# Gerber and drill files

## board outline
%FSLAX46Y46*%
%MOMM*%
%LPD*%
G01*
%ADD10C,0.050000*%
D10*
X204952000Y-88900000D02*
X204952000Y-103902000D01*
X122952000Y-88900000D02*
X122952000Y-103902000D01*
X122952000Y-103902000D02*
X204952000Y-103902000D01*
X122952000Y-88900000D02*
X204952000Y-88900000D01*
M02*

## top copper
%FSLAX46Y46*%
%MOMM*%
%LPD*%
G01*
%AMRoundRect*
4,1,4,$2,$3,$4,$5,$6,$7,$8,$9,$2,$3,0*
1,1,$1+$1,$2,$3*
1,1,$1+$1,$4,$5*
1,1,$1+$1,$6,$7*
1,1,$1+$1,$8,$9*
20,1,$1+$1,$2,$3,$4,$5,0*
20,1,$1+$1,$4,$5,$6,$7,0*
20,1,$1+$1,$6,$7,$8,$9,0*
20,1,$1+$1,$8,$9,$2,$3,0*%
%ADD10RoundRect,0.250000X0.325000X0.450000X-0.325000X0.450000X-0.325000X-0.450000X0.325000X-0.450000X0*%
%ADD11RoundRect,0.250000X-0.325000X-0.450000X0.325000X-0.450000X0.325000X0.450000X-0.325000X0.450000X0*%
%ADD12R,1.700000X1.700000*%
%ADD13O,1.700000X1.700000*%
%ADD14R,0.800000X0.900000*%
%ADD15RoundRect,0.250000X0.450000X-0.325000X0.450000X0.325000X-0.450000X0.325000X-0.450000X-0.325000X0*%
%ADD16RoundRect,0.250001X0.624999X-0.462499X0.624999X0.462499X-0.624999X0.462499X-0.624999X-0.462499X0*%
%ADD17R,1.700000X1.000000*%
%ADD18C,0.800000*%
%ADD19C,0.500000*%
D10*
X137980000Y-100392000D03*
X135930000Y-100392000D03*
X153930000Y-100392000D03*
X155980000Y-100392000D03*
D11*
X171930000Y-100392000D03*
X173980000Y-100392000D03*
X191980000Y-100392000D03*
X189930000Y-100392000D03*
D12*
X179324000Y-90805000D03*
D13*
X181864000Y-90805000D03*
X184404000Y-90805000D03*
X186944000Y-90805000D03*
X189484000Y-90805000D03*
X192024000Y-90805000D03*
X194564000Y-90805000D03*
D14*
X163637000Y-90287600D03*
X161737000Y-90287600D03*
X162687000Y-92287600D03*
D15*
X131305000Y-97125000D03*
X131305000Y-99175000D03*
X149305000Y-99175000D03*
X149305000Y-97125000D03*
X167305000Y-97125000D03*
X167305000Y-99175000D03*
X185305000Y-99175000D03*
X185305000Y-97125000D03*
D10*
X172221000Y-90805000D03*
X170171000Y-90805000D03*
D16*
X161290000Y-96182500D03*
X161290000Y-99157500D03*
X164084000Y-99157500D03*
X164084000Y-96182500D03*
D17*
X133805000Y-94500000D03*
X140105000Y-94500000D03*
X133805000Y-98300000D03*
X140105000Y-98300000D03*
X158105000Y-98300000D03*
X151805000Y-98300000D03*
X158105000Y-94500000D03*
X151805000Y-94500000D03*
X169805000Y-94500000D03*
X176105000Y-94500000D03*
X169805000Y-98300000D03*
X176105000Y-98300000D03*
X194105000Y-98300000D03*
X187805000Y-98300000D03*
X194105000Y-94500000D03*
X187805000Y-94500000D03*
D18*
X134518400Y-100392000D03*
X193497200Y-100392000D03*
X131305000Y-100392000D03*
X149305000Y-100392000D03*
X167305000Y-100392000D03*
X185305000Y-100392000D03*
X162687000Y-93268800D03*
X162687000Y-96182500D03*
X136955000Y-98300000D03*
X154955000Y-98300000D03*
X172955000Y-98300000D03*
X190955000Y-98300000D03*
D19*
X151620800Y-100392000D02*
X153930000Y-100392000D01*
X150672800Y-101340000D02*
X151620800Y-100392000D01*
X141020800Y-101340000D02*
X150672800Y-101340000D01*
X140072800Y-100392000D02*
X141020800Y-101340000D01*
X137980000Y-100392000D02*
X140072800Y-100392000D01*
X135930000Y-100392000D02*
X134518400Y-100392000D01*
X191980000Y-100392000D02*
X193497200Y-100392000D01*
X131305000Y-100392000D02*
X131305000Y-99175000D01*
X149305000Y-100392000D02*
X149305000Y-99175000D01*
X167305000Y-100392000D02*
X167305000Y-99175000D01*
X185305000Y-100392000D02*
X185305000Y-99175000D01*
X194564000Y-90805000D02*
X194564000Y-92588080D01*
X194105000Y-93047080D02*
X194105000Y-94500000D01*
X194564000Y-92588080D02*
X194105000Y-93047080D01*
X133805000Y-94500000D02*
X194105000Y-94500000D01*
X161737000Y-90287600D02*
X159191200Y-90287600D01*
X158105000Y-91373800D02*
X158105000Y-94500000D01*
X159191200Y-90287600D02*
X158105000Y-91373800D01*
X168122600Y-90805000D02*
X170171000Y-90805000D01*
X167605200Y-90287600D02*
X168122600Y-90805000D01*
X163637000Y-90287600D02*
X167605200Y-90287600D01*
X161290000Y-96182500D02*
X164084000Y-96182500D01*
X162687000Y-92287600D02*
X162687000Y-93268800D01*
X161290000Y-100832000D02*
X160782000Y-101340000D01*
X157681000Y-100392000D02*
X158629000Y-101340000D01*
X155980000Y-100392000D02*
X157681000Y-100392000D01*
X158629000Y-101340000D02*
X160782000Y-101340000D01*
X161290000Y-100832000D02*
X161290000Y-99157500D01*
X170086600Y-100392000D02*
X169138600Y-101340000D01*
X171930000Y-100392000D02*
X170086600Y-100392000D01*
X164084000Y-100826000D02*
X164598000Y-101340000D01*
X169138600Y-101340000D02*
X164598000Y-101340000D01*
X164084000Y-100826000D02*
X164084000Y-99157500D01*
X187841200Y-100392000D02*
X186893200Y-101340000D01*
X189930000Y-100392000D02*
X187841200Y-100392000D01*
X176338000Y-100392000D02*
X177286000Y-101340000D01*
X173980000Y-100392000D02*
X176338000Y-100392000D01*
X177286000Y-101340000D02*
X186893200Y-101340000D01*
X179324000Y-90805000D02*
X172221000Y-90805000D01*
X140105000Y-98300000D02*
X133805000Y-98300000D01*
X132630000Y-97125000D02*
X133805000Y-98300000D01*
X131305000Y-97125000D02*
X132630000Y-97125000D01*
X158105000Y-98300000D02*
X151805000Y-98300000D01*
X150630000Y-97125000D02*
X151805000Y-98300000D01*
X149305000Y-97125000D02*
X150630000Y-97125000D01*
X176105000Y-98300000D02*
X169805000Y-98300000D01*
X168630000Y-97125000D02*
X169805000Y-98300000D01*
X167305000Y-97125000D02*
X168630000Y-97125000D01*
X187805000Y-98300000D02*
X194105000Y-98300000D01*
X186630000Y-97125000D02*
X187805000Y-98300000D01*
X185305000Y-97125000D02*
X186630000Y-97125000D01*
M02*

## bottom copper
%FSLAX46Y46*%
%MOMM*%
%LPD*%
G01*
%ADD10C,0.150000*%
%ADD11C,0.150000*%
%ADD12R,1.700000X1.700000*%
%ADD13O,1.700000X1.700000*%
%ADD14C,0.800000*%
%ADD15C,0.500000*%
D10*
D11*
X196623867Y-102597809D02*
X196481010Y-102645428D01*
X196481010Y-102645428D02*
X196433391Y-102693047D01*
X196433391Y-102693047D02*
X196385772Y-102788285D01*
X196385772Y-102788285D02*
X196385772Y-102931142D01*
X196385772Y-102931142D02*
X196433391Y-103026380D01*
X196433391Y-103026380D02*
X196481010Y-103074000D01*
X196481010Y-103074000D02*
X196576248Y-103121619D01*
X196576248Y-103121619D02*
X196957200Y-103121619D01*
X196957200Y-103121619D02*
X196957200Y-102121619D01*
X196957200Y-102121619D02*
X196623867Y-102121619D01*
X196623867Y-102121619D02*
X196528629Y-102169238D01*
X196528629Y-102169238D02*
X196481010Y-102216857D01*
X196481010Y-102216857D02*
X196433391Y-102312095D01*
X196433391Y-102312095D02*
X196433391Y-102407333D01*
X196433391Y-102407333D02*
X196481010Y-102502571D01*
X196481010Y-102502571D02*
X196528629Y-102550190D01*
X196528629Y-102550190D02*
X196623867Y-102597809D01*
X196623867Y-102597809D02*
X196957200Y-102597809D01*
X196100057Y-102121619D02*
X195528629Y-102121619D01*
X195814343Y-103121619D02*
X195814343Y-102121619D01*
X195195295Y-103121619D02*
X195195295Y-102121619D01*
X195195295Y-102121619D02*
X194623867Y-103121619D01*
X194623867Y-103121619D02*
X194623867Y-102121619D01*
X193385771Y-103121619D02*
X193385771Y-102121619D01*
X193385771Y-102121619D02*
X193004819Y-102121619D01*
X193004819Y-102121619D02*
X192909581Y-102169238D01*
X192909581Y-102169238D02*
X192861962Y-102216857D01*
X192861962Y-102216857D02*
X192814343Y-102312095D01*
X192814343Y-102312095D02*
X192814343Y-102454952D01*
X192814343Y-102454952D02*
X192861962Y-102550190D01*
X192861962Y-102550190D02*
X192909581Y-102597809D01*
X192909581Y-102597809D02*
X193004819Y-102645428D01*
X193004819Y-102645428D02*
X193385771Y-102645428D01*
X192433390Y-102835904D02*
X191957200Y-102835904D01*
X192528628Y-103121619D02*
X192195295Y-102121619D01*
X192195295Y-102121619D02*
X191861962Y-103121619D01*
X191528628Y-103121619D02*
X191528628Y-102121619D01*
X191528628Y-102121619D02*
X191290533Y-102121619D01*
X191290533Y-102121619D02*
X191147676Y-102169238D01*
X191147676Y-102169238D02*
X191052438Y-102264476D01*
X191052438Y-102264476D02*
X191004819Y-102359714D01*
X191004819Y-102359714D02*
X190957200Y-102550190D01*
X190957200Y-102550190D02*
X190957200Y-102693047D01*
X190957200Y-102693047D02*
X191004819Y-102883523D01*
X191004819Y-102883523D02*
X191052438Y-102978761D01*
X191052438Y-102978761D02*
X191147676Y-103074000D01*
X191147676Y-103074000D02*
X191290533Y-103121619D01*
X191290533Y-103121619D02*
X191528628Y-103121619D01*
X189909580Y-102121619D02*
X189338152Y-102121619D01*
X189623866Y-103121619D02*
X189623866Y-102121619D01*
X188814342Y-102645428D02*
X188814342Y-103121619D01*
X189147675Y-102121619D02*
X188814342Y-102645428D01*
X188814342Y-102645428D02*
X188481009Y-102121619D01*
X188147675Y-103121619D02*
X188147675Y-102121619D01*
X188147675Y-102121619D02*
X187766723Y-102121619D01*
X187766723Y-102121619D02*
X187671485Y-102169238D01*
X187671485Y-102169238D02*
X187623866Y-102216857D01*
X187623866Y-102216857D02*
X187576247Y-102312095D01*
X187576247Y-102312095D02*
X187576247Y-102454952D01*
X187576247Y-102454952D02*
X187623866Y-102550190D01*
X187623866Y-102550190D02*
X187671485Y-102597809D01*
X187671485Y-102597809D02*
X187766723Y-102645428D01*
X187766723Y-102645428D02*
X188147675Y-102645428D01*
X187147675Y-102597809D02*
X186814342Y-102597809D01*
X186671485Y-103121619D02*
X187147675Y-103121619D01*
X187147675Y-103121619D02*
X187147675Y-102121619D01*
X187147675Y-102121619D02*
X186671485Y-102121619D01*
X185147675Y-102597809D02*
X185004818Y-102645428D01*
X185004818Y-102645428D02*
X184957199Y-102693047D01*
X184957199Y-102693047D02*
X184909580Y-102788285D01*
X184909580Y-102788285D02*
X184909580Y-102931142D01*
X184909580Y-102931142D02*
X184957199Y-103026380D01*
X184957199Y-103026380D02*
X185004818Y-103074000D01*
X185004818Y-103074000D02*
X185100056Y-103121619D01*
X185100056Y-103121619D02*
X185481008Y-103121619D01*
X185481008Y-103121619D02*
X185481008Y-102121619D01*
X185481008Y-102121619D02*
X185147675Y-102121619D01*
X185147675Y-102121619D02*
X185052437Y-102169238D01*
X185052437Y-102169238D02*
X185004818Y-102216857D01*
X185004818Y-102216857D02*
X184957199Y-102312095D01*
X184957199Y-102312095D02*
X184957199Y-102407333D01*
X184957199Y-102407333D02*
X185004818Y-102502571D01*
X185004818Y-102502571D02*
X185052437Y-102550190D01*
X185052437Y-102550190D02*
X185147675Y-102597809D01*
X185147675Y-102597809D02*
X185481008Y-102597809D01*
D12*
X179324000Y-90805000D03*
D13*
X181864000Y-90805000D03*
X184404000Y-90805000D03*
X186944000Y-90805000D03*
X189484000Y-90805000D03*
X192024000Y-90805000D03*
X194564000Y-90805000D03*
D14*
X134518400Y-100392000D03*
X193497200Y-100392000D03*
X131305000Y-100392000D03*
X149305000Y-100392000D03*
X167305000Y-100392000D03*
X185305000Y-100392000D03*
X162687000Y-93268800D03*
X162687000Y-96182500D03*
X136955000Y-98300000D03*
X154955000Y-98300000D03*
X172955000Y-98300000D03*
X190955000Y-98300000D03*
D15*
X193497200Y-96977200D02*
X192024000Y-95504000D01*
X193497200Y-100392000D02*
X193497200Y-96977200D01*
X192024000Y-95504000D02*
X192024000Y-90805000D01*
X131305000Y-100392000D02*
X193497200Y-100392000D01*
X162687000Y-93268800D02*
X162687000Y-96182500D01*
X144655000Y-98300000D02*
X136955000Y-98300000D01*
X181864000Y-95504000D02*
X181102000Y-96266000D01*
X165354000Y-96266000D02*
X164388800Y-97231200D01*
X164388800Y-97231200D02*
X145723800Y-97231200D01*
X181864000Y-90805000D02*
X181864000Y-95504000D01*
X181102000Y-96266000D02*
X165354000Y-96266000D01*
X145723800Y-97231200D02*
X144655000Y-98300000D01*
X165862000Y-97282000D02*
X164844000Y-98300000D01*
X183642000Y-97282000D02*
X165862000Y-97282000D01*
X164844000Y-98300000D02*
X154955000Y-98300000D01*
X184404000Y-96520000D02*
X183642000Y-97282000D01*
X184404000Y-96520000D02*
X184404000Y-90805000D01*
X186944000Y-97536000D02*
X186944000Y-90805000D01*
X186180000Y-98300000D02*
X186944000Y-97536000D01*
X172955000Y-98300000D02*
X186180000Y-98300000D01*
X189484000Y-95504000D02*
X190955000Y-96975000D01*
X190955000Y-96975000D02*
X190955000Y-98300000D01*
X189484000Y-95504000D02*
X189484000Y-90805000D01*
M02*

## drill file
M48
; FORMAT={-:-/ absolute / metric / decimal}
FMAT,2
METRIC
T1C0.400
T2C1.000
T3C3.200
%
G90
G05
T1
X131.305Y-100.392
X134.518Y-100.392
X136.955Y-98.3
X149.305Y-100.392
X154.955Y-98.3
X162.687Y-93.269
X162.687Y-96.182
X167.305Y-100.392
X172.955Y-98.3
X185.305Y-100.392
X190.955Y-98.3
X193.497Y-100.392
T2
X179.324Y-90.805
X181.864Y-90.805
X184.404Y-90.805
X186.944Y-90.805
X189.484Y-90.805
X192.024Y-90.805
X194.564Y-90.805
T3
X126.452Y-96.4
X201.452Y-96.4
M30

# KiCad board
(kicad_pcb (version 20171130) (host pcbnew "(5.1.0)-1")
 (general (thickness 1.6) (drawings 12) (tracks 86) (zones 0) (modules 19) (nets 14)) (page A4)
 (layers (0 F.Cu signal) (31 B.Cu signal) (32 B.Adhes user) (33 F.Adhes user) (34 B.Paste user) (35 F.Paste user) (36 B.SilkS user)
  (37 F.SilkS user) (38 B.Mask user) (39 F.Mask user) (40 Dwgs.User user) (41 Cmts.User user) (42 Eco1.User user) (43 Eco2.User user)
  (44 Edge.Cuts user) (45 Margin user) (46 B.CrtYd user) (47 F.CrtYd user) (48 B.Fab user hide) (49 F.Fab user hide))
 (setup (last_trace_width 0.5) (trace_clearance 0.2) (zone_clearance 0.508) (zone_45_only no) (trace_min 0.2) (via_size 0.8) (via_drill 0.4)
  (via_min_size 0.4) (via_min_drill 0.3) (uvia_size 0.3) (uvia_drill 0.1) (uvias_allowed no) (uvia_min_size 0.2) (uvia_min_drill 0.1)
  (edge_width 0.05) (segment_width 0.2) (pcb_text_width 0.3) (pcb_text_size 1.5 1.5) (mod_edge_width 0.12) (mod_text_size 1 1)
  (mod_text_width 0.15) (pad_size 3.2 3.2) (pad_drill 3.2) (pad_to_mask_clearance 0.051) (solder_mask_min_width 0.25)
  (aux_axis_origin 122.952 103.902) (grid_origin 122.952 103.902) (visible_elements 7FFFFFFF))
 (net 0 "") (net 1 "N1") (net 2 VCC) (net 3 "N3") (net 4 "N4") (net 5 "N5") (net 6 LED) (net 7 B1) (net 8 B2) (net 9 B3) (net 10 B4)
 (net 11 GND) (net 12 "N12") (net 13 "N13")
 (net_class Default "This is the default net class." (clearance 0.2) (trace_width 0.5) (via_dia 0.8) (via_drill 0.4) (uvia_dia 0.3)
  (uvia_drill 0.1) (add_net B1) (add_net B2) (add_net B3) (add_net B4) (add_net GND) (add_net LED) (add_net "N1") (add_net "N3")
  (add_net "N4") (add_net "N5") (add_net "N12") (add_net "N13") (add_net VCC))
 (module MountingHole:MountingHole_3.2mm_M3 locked (layer F.Cu) (at 201.452 96.4)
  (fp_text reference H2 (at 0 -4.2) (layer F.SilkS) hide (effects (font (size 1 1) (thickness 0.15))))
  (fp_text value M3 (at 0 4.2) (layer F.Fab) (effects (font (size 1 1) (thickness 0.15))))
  (pad 1 np_thru_hole circle (at 0 0) (size 3.2 3.2) (drill 3.2) (layers *.Cu *.Mask)))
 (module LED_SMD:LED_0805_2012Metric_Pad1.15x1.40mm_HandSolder (layer F.Cu) (at 136.955 100.392 180)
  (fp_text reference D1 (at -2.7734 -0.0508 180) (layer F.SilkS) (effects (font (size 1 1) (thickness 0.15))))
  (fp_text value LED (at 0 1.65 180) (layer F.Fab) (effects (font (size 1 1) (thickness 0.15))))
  (pad 1 smd roundrect (at -1.025 0 180) (size 1.15 1.4) (layers F.Cu F.Paste F.Mask) (roundrect_rratio 0.217391) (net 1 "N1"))
  (pad 2 smd roundrect (at 1.025 0 180) (size 1.15 1.4) (layers F.Cu F.Paste F.Mask) (roundrect_rratio 0.217391) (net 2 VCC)))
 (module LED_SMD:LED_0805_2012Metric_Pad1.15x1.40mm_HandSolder (layer F.Cu) (at 154.955 100.392 180)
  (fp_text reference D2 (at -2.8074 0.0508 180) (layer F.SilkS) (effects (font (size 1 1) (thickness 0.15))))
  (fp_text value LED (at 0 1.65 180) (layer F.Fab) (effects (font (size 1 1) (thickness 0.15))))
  (pad 2 smd roundrect (at 1.025 0 180) (size 1.15 1.4) (layers F.Cu F.Paste F.Mask) (roundrect_rratio 0.217391) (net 1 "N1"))
  (pad 1 smd roundrect (at -1.025 0 180) (size 1.15 1.4) (layers F.Cu F.Paste F.Mask) (roundrect_rratio 0.217391) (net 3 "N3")))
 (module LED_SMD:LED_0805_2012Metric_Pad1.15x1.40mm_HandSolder (layer F.Cu) (at 172.955 100.392)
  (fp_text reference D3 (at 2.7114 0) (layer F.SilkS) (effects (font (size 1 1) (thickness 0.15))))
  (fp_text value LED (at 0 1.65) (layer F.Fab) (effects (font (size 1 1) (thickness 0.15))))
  (pad 1 smd roundrect (at -1.025 0) (size 1.15 1.4) (layers F.Cu F.Paste F.Mask) (roundrect_rratio 0.217391) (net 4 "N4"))
  (pad 2 smd roundrect (at 1.025 0) (size 1.15 1.4) (layers F.Cu F.Paste F.Mask) (roundrect_rratio 0.217391) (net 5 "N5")))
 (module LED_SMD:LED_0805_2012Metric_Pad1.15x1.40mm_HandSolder (layer F.Cu) (at 190.955 100.392)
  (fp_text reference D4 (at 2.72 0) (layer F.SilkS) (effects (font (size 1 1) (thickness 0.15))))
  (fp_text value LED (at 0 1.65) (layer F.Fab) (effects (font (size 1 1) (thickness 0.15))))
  (pad 2 smd roundrect (at 1.025 0) (size 1.15 1.4) (layers F.Cu F.Paste F.Mask) (roundrect_rratio 0.217391) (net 2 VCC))
  (pad 1 smd roundrect (at -1.025 0) (size 1.15 1.4) (layers F.Cu F.Paste F.Mask) (roundrect_rratio 0.217391) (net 5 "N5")))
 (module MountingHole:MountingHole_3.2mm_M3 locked (layer F.Cu) (at 126.452 96.4)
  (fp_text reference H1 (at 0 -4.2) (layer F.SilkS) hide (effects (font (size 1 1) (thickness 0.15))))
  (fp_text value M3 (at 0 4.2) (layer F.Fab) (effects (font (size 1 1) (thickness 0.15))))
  (pad "" np_thru_hole circle (at 0 0) (size 3.2 3.2) (drill 3.2) (layers *.Cu *.Mask)))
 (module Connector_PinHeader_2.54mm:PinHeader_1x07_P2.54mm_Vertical (layer B.Cu) (at 179.324 90.805 270)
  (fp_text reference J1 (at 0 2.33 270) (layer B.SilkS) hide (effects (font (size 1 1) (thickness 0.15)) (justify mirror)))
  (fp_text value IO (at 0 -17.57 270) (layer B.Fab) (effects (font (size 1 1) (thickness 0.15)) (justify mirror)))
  (pad 1 thru_hole rect (at 0 0 270) (size 1.7 1.7) (drill 1) (layers *.Cu *.Mask) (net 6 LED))
  (pad 2 thru_hole oval (at 0 -2.54 270) (size 1.7 1.7) (drill 1) (layers *.Cu *.Mask) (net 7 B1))
  (pad 3 thru_hole oval (at 0 -5.08 270) (size 1.7 1.7) (drill 1) (layers *.Cu *.Mask) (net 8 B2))
  (pad 4 thru_hole oval (at 0 -7.62 270) (size 1.7 1.7) (drill 1) (layers *.Cu *.Mask) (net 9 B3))
  (pad 5 thru_hole oval (at 0 -10.16 270) (size 1.7 1.7) (drill 1) (layers *.Cu *.Mask) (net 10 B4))
  (pad 6 thru_hole oval (at 0 -12.7 270) (size 1.7 1.7) (drill 1) (layers *.Cu *.Mask) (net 2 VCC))
  (pad 7 thru_hole oval (at 0 -15.24 270) (size 1.7 1.7) (drill 1) (layers *.Cu *.Mask) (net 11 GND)))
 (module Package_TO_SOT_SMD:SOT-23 (layer F.Cu) (at 162.687 91.2876 270)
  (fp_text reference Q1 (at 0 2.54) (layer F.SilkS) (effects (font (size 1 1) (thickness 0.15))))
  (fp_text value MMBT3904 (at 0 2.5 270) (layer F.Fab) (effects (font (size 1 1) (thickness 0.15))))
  (pad 1 smd rect (at -1 -0.95 270) (size 0.9 0.8) (layers F.Cu F.Paste F.Mask) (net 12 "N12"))
  (pad 2 smd rect (at -1 0.95 270) (size 0.9 0.8) (layers F.Cu F.Paste F.Mask) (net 11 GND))
  (pad 3 smd rect (at 1 0 270) (size 0.9 0.8) (layers F.Cu F.Paste F.Mask) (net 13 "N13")))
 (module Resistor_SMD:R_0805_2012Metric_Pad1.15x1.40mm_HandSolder (layer F.Cu) (at 131.305 98.15 90)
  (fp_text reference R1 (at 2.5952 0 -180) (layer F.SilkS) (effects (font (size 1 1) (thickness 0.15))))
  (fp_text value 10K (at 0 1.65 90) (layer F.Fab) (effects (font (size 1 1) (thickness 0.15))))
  (pad 2 smd roundrect (at 1.025 0 90) (size 1.15 1.4) (layers F.Cu F.Paste F.Mask) (roundrect_rratio 0.217391) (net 7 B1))
  (pad 1 smd roundrect (at -1.025 0 90) (size 1.15 1.4) (layers F.Cu F.Paste F.Mask) (roundrect_rratio 0.217391) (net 2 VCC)))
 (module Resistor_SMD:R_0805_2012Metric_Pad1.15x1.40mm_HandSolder (layer F.Cu) (at 149.305 98.15 90)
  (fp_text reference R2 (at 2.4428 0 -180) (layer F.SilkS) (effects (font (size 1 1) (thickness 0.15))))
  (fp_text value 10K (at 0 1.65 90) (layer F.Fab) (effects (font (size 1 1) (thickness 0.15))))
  (pad 1 smd roundrect (at -1.025 0 90) (size 1.15 1.4) (layers F.Cu F.Paste F.Mask) (roundrect_rratio 0.217391) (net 2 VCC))
  (pad 2 smd roundrect (at 1.025 0 90) (size 1.15 1.4) (layers F.Cu F.Paste F.Mask) (roundrect_rratio 0.217391) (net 8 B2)))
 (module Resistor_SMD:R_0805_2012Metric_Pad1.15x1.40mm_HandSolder (layer F.Cu) (at 167.305 98.15 90)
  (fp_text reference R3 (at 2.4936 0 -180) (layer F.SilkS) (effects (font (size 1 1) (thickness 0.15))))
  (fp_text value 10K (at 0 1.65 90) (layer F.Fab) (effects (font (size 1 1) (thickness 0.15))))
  (pad 2 smd roundrect (at 1.025 0 90) (size 1.15 1.4) (layers F.Cu F.Paste F.Mask) (roundrect_rratio 0.217391) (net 9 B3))
  (pad 1 smd roundrect (at -1.025 0 90) (size 1.15 1.4) (layers F.Cu F.Paste F.Mask) (roundrect_rratio 0.217391) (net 2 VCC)))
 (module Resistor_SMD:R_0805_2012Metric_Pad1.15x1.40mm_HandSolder (layer F.Cu) (at 185.305 98.15 90)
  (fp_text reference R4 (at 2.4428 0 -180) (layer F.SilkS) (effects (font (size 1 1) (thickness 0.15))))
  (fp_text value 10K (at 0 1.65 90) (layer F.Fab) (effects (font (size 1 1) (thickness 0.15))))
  (pad 1 smd roundrect (at -1.025 0 90) (size 1.15 1.4) (layers F.Cu F.Paste F.Mask) (roundrect_rratio 0.217391) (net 2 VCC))
  (pad 2 smd roundrect (at 1.025 0 90) (size 1.15 1.4) (layers F.Cu F.Paste F.Mask) (roundrect_rratio 0.217391) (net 10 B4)))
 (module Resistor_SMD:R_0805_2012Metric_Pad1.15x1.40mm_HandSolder (layer F.Cu) (at 171.196 90.805 180)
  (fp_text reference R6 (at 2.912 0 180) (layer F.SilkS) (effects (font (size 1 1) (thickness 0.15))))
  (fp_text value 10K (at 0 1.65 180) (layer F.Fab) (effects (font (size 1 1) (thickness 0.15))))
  (pad 1 smd roundrect (at -1.025 0 180) (size 1.15 1.4) (layers F.Cu F.Paste F.Mask) (roundrect_rratio 0.217391) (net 6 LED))
  (pad 2 smd roundrect (at 1.025 0 180) (size 1.15 1.4) (layers F.Cu F.Paste F.Mask) (roundrect_rratio 0.217391) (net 12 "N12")))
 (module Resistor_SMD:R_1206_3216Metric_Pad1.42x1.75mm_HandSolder (layer F.Cu) (at 161.29 97.67 90)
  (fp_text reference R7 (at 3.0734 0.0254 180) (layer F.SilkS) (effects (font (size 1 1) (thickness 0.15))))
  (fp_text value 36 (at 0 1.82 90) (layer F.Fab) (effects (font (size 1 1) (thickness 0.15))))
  (pad 2 smd roundrect (at 1.4875 0 90) (size 1.425 1.75) (layers F.Cu F.Paste F.Mask) (roundrect_rratio 0.175439) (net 13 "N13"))
  (pad 1 smd roundrect (at -1.4875 0 90) (size 1.425 1.75) (layers F.Cu F.Paste F.Mask) (roundrect_rratio 0.175439) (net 3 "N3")))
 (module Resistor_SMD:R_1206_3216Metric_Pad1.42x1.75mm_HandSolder (layer F.Cu) (at 164.084 97.67 90)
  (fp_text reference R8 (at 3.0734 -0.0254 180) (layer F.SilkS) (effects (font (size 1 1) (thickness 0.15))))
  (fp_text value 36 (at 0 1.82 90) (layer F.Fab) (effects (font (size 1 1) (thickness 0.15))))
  (pad 1 smd roundrect (at -1.4875 0 90) (size 1.425 1.75) (layers F.Cu F.Paste F.Mask) (roundrect_rratio 0.175439) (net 4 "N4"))
  (pad 2 smd roundrect (at 1.4875 0 90) (size 1.425 1.75) (layers F.Cu F.Paste F.Mask) (roundrect_rratio 0.175439) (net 13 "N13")))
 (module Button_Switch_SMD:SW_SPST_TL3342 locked (layer F.Cu) (at 136.955 96.4)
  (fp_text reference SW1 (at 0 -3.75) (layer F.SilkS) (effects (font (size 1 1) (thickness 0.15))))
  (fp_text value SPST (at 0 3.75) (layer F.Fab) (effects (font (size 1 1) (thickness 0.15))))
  (pad 1 smd rect (at -3.15 -1.9) (size 1.7 1) (layers F.Cu F.Paste F.Mask) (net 11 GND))
  (pad 1 smd rect (at 3.15 -1.9) (size 1.7 1) (layers F.Cu F.Paste F.Mask) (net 11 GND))
  (pad 2 smd rect (at -3.15 1.9) (size 1.7 1) (layers F.Cu F.Paste F.Mask) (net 7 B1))
  (pad 2 smd rect (at 3.15 1.9) (size 1.7 1) (layers F.Cu F.Paste F.Mask) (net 7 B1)))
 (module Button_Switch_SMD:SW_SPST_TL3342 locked (layer F.Cu) (at 154.955 96.4)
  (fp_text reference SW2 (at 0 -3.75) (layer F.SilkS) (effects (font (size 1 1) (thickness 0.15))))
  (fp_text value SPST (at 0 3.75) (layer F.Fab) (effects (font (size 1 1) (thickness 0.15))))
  (pad 2 smd rect (at 3.15 1.9) (size 1.7 1) (layers F.Cu F.Paste F.Mask) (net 8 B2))
  (pad 2 smd rect (at -3.15 1.9) (size 1.7 1) (layers F.Cu F.Paste F.Mask) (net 8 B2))
  (pad 1 smd rect (at 3.15 -1.9) (size 1.7 1) (layers F.Cu F.Paste F.Mask) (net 11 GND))
  (pad 1 smd rect (at -3.15 -1.9) (size 1.7 1) (layers F.Cu F.Paste F.Mask) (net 11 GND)))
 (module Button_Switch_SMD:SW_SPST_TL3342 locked (layer F.Cu) (at 172.955 96.4)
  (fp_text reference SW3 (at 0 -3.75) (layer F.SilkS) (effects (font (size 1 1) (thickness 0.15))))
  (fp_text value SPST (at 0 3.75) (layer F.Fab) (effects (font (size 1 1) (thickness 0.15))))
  (pad 1 smd rect (at -3.15 -1.9) (size 1.7 1) (layers F.Cu F.Paste F.Mask) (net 11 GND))
  (pad 1 smd rect (at 3.15 -1.9) (size 1.7 1) (layers F.Cu F.Paste F.Mask) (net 11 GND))
  (pad 2 smd rect (at -3.15 1.9) (size 1.7 1) (layers F.Cu F.Paste F.Mask) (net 9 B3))
  (pad 2 smd rect (at 3.15 1.9) (size 1.7 1) (layers F.Cu F.Paste F.Mask) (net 9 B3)))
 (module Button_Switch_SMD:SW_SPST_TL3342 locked (layer F.Cu) (at 190.955 96.4)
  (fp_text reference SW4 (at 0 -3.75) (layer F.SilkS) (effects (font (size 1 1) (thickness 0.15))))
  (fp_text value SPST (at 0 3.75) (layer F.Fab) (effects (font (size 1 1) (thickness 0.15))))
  (pad 2 smd rect (at 3.15 1.9) (size 1.7 1) (layers F.Cu F.Paste F.Mask) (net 10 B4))
  (pad 2 smd rect (at -3.15 1.9) (size 1.7 1) (layers F.Cu F.Paste F.Mask) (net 10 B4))
  (pad 1 smd rect (at 3.15 -1.9) (size 1.7 1) (layers F.Cu F.Paste F.Mask) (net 11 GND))
  (pad 1 smd rect (at -3.15 -1.9) (size 1.7 1) (layers F.Cu F.Paste F.Mask) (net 11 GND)))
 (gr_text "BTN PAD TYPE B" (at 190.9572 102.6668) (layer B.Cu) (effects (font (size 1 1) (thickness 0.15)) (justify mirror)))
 (gr_line (start 204.952 88.9) (end 204.952 103.902) (layer Edge.Cuts) (width 0.05))
 (gr_line (start 122.952 88.9) (end 122.952 103.902) (layer Edge.Cuts) (width 0.05))
 (gr_line (start 122.952 103.902) (end 204.952 103.902) (layer Edge.Cuts) (width 0.05))
 (gr_line (start 122.952 88.9) (end 204.952 88.9) (layer Edge.Cuts) (width 0.05))
 (segment (start 151.6208 100.392) (end 153.93 100.392) (width 0.5) (layer F.Cu) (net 1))
 (segment (start 150.6728 101.34) (end 151.6208 100.392) (width 0.5) (layer F.Cu) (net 1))
 (segment (start 141.0208 101.34) (end 150.6728 101.34) (width 0.5) (layer F.Cu) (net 1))
 (segment (start 140.0728 100.392) (end 141.0208 101.34) (width 0.5) (layer F.Cu) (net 1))
 (segment (start 137.98 100.392) (end 140.0728 100.392) (width 0.5) (layer F.Cu) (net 1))
 (via (at 134.5184 100.392) (size 0.8) (drill 0.4) (layers F.Cu B.Cu) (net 2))
 (segment (start 135.93 100.392) (end 134.5184 100.392) (width 0.5) (layer F.Cu) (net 2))
 (segment (start 191.98 100.392) (end 193.4972 100.392) (width 0.5) (layer F.Cu) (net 2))
 (via (at 193.4972 100.392) (size 0.8) (drill 0.4) (layers F.Cu B.Cu) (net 2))
 (via (at 131.305 100.392) (size 0.8) (drill 0.4) (layers F.Cu B.Cu) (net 2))
 (via (at 149.305 100.392) (size 0.8) (drill 0.4) (layers F.Cu B.Cu) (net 2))
 (via (at 167.305 100.392) (size 0.8) (drill 0.4) (layers F.Cu B.Cu) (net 2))
 (via (at 185.305 100.392) (size 0.8) (drill 0.4) (layers F.Cu B.Cu) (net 2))
 (segment (start 193.4972 96.9772) (end 192.024 95.504) (width 0.5) (layer B.Cu) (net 2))
 (segment (start 193.4972 100.392) (end 193.4972 96.9772) (width 0.5) (layer B.Cu) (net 2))
 (segment (start 192.024 95.504) (end 192.024 90.805) (width 0.5) (layer B.Cu) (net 2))
 (segment (start 131.305 100.392) (end 131.305 99.175) (width 0.5) (layer F.Cu) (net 2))
 (segment (start 149.305 100.392) (end 149.305 99.175) (width 0.5) (layer F.Cu) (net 2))
 (segment (start 167.305 100.392) (end 167.305 99.175) (width 0.5) (layer F.Cu) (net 2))
 (segment (start 185.305 100.392) (end 185.305 99.175) (width 0.5) (layer F.Cu) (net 2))
 (segment (start 131.305 100.392) (end 193.4972 100.392) (width 0.5) (layer B.Cu) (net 2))
 (segment (start 194.564 90.805) (end 194.564 92.58808) (width 0.5) (layer F.Cu) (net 11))
 (segment (start 194.105 93.04708) (end 194.105 94.5) (width 0.5) (layer F.Cu) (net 11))
 (segment (start 194.564 92.58808) (end 194.105 93.04708) (width 0.5) (layer F.Cu) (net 11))
 (segment (start 133.805 94.5) (end 194.105 94.5) (width 0.5) (layer F.Cu) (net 11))
 (segment (start 161.737 90.2876) (end 159.1912 90.2876) (width 0.5) (layer F.Cu) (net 11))
 (segment (start 158.105 91.3738) (end 158.105 94.5) (width 0.5) (layer F.Cu) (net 11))
 (segment (start 159.1912 90.2876) (end 158.105 91.3738) (width 0.5) (layer F.Cu) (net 11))
 (segment (start 168.1226 90.805) (end 170.171 90.805) (width 0.5) (layer F.Cu) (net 12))
 (segment (start 167.6052 90.2876) (end 168.1226 90.805) (width 0.5) (layer F.Cu) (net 12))
 (segment (start 163.637 90.2876) (end 167.6052 90.2876) (width 0.5) (layer F.Cu) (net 12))
 (via (at 162.687 93.2688) (size 0.8) (drill 0.4) (layers F.Cu B.Cu) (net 13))
 (segment (start 161.29 96.1825) (end 164.084 96.1825) (width 0.5) (layer F.Cu) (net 13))
 (via (at 162.687 96.1825) (size 0.8) (drill 0.4) (layers F.Cu B.Cu) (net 13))
 (segment (start 162.687 92.2876) (end 162.687 93.2688) (width 0.5) (layer F.Cu) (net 13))
 (segment (start 162.687 93.2688) (end 162.687 96.1825) (width 0.5) (layer B.Cu) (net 13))
 (segment (start 161.29 100.832) (end 160.782 101.34) (width 0.5) (layer F.Cu) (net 3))
 (segment (start 157.681 100.392) (end 158.629 101.34) (width 0.5) (layer F.Cu) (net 3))
 (segment (start 155.98 100.392) (end 157.681 100.392) (width 0.5) (layer F.Cu) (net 3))
 (segment (start 158.629 101.34) (end 160.782 101.34) (width 0.5) (layer F.Cu) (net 3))
 (segment (start 161.29 100.832) (end 161.29 99.1575) (width 0.5) (layer F.Cu) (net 3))
 (segment (start 170.0866 100.392) (end 169.1386 101.34) (width 0.5) (layer F.Cu) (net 4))
 (segment (start 171.93 100.392) (end 170.0866 100.392) (width 0.5) (layer F.Cu) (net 4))
 (segment (start 164.084 100.826) (end 164.598 101.34) (width 0.5) (layer F.Cu) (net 4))
 (segment (start 169.1386 101.34) (end 164.598 101.34) (width 0.5) (layer F.Cu) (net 4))
 (segment (start 164.084 100.826) (end 164.084 99.1575) (width 0.5) (layer F.Cu) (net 4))
 (segment (start 187.8412 100.392) (end 186.8932 101.34) (width 0.5) (layer F.Cu) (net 5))
 (segment (start 189.93 100.392) (end 187.8412 100.392) (width 0.5) (layer F.Cu) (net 5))
 (segment (start 176.338 100.392) (end 177.286 101.34) (width 0.5) (layer F.Cu) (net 5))
 (segment (start 173.98 100.392) (end 176.338 100.392) (width 0.5) (layer F.Cu) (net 5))
 (segment (start 177.286 101.34) (end 186.8932 101.34) (width 0.5) (layer F.Cu) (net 5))
 (segment (start 179.324 90.805) (end 172.221 90.805) (width 0.5) (layer F.Cu) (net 6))
 (segment (start 140.105 98.3) (end 133.805 98.3) (width 0.5) (layer F.Cu) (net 7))
 (via (at 136.955 98.3) (size 0.8) (drill 0.4) (layers F.Cu B.Cu) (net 7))
 (segment (start 144.655 98.3) (end 136.955 98.3) (width 0.5) (layer B.Cu) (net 7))
 (segment (start 181.864 95.504) (end 181.102 96.266) (width 0.5) (layer B.Cu) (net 7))
 (segment (start 165.354 96.266) (end 164.3888 97.2312) (width 0.5) (layer B.Cu) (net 7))
 (segment (start 164.3888 97.2312) (end 145.7238 97.2312) (width 0.5) (layer B.Cu) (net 7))
 (segment (start 181.864 90.805) (end 181.864 95.504) (width 0.5) (layer B.Cu) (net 7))
 (segment (start 181.102 96.266) (end 165.354 96.266) (width 0.5) (layer B.Cu) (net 7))
 (segment (start 145.7238 97.2312) (end 144.655 98.3) (width 0.5) (layer B.Cu) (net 7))
 (segment (start 132.63 97.125) (end 133.805 98.3) (width 0.5) (layer F.Cu) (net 7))
 (segment (start 131.305 97.125) (end 132.63 97.125) (width 0.5) (layer F.Cu) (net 7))
 (segment (start 158.105 98.3) (end 151.805 98.3) (width 0.5) (layer F.Cu) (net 8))
 (via (at 154.955 98.3) (size 0.8) (drill 0.4) (layers F.Cu B.Cu) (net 8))
 (segment (start 165.862 97.282) (end 164.844 98.3) (width 0.5) (layer B.Cu) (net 8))
 (segment (start 183.642 97.282) (end 165.862 97.282) (width 0.5) (layer B.Cu) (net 8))
 (segment (start 164.844 98.3) (end 154.955 98.3) (width 0.5) (layer B.Cu) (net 8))
 (segment (start 184.404 96.52) (end 183.642 97.282) (width 0.5) (layer B.Cu) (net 8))
 (segment (start 184.404 96.52) (end 184.404 90.805) (width 0.5) (layer B.Cu) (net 8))
 (segment (start 150.63 97.125) (end 151.805 98.3) (width 0.5) (layer F.Cu) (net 8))
 (segment (start 149.305 97.125) (end 150.63 97.125) (width 0.5) (layer F.Cu) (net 8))
 (segment (start 176.105 98.3) (end 169.805 98.3) (width 0.5) (layer F.Cu) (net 9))
 (via (at 172.955 98.3) (size 0.8) (drill 0.4) (layers F.Cu B.Cu) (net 9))
 (segment (start 186.944 97.536) (end 186.944 90.805) (width 0.5) (layer B.Cu) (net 9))
 (segment (start 186.18 98.3) (end 186.944 97.536) (width 0.5) (layer B.Cu) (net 9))
 (segment (start 172.955 98.3) (end 186.18 98.3) (width 0.5) (layer B.Cu) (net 9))
 (segment (start 168.63 97.125) (end 169.805 98.3) (width 0.5) (layer F.Cu) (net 9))
 (segment (start 167.305 97.125) (end 168.63 97.125) (width 0.5) (layer F.Cu) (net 9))
 (segment (start 187.805 98.3) (end 194.105 98.3) (width 0.5) (layer F.Cu) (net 10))
 (via (at 190.955 98.3) (size 0.8) (drill 0.4) (layers F.Cu B.Cu) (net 10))
 (segment (start 189.484 95.504) (end 190.955 96.975) (width 0.5) (layer B.Cu) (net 10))
 (segment (start 190.955 96.975) (end 190.955 98.3) (width 0.5) (layer B.Cu) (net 10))
 (segment (start 189.484 95.504) (end 189.484 90.805) (width 0.5) (layer B.Cu) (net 10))
 (segment (start 186.63 97.125) (end 187.805 98.3) (width 0.5) (layer F.Cu) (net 10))
 (segment (start 185.305 97.125) (end 186.63 97.125) (width 0.5) (layer F.Cu) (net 10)))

